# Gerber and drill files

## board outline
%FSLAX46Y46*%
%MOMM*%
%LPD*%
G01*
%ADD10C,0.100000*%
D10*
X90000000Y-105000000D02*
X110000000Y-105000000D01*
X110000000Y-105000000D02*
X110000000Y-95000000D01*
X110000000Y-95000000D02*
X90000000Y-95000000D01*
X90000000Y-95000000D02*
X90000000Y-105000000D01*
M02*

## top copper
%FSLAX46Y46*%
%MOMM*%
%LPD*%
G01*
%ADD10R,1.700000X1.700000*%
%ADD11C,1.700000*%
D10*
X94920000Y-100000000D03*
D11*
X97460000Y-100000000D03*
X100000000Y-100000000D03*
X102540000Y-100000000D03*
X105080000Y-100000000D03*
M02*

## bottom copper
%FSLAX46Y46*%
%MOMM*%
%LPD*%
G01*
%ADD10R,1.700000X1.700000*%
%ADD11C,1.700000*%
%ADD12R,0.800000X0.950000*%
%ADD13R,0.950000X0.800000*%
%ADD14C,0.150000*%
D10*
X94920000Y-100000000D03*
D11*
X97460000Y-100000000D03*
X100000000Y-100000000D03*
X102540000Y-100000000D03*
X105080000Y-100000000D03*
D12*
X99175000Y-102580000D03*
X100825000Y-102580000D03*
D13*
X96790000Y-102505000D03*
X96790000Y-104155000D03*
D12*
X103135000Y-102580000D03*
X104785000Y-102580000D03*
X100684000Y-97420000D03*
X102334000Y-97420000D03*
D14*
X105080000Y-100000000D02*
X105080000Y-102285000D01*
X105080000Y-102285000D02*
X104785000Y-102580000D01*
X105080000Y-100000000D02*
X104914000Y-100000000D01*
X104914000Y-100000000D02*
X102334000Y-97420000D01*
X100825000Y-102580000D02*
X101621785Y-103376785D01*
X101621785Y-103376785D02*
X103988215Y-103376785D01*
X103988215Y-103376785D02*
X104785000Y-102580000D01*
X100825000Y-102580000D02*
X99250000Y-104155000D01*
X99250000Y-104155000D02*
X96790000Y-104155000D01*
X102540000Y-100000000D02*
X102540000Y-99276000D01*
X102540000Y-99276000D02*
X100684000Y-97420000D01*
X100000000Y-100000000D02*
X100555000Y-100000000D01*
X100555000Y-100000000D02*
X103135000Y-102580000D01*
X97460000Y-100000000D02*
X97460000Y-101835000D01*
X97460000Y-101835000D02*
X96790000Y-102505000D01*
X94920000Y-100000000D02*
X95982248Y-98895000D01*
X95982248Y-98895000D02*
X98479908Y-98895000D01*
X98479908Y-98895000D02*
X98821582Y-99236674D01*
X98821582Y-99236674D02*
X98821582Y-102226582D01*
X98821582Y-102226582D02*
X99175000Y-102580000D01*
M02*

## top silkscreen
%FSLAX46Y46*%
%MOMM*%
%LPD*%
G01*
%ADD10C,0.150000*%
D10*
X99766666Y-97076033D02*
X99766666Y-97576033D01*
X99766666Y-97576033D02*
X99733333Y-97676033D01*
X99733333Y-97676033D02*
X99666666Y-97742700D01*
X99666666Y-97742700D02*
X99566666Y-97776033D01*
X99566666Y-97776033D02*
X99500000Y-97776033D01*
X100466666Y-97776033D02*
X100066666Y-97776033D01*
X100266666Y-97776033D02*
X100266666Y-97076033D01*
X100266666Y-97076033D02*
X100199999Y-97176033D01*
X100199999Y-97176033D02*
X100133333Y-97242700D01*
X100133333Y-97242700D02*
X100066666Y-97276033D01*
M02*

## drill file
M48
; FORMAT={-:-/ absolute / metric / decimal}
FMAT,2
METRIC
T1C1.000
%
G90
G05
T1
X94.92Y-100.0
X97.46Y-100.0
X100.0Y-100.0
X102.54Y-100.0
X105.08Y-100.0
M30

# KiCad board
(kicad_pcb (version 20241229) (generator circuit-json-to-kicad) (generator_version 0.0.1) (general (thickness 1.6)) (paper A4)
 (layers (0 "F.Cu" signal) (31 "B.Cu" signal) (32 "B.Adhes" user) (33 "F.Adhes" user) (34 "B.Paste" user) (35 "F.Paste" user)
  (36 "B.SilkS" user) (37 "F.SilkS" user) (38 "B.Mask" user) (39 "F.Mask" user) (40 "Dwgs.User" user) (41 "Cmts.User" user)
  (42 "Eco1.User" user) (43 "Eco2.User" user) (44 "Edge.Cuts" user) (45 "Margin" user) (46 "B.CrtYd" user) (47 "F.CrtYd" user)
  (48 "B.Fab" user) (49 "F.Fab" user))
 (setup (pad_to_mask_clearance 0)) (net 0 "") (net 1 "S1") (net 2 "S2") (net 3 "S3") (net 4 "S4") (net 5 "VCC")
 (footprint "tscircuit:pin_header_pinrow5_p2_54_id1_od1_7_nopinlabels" (layer F.Cu) (at 100 100 0)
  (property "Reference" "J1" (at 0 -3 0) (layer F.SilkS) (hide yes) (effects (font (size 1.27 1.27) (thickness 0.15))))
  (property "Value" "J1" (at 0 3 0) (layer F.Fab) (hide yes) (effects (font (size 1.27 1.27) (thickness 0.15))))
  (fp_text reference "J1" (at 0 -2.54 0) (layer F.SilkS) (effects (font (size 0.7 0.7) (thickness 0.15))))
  (pad "1" thru_hole rect (at -5.08 0 0) (size 1.7 1.7) (drill 1) (layers *.Cu *.Mask) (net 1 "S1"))
  (pad "2" thru_hole circle (at -2.54 0 0) (size 1.7 1.7) (drill 1) (layers *.Cu *.Mask) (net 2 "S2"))
  (pad "3" thru_hole circle (at 0 0 0) (size 1.7 1.7) (drill 1) (layers *.Cu *.Mask) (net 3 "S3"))
  (pad "4" thru_hole circle (at 2.54 0 0) (size 1.7 1.7) (drill 1) (layers *.Cu *.Mask) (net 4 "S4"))
  (pad "5" thru_hole circle (at 5.08 0 0) (size 1.7 1.7) (drill 1) (layers *.Cu *.Mask) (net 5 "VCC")))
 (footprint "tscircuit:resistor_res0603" (layer B.Cu) (at 100 102.58 180)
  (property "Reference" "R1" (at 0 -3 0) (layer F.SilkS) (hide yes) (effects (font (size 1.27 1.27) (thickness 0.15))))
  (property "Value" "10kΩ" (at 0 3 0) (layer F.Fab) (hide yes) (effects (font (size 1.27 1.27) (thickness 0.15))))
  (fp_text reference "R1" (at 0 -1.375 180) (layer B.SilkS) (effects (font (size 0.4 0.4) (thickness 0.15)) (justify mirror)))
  (pad "1" smd rect (at 0.825 0 0) (size 0.8 0.95) (layers B.Cu B.Mask) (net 1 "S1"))
  (pad "2" smd rect (at -0.825 0 0) (size 0.8 0.95) (layers B.Cu B.Mask) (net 5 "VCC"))
  (pad "" smd rect (at 0.825 0 0) (size 0.5599999999999999 0.6649999999999999) (layers B.Paste))
  (pad "" smd rect (at -0.825 0 0) (size 0.5599999999999999 0.6649999999999999) (layers B.Paste)))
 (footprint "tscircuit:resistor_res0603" (layer B.Cu) (at 96.79 103.33 90)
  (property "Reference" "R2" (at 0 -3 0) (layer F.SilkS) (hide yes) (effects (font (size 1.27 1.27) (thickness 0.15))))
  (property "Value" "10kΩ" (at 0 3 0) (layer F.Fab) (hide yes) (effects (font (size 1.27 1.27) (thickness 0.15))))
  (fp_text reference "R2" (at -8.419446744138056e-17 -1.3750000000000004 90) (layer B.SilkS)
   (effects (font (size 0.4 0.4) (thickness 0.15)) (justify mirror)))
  (pad "1" smd rect (at 0.8249999999999997 0 0) (size 0.95 0.8) (layers B.Cu B.Mask) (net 2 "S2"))
  (pad "2" smd rect (at -0.8249999999999997 4.440892098500626e-16 0) (size 0.95 0.8) (layers B.Cu B.Mask) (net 5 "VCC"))
  (pad "" smd rect (at 0.8249999999999997 0 0) (size 0.6649999999999999 0.5599999999999999) (layers B.Paste))
  (pad "" smd rect (at -0.8249999999999997 4.440892098500626e-16 0) (size 0.6649999999999999 0.5599999999999999) (layers B.Paste)))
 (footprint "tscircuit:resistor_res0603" (layer B.Cu) (at 103.96 102.58 180)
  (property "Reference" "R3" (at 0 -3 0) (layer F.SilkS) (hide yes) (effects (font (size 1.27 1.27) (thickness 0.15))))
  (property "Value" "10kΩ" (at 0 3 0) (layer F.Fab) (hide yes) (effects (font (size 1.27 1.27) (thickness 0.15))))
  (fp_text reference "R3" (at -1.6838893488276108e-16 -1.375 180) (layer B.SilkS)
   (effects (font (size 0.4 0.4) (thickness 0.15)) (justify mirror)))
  (pad "1" smd rect (at 0.8250000000000002 0 0) (size 0.8 0.95) (layers B.Cu B.Mask) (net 3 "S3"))
  (pad "2" smd rect (at -0.8249999999999997 0 0) (size 0.8 0.95) (layers B.Cu B.Mask) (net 5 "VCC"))
  (pad "" smd rect (at 0.8250000000000002 0 0) (size 0.5599999999999999 0.6649999999999999) (layers B.Paste))
  (pad "" smd rect (at -0.8249999999999997 0 0) (size 0.5599999999999999 0.6649999999999999) (layers B.Paste)))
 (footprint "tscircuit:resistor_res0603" (layer B.Cu) (at 101.509 97.42 180)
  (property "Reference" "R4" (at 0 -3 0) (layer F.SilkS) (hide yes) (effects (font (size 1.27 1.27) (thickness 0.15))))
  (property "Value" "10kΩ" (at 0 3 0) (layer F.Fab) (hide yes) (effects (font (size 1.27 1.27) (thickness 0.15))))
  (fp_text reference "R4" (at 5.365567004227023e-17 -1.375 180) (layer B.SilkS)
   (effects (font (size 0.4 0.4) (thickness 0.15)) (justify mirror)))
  (pad "1" smd rect (at 0.8250000000000001 0 0) (size 0.8 0.95) (layers B.Cu B.Mask) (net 4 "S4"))
  (pad "2" smd rect (at -0.825 4.440892098500626e-16 0) (size 0.8 0.95) (layers B.Cu B.Mask) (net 5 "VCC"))
  (pad "" smd rect (at 0.8250000000000001 0 0) (size 0.5599999999999999 0.6649999999999999) (layers B.Paste))
  (pad "" smd rect (at -0.825 4.440892098500626e-16 0) (size 0.5599999999999999 0.6649999999999999) (layers B.Paste)))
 (segment (start 105.08 100) (end 105.08 102.285) (width 0.15) (layer B.Cu) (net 5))
 (segment (start 105.08 102.285) (end 104.785 102.58) (width 0.15) (layer B.Cu) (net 5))
 (segment (start 105.08 100) (end 104.914 100) (width 0.15) (layer B.Cu) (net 5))
 (segment (start 104.914 100) (end 102.334 97.42) (width 0.15) (layer B.Cu) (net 5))
 (segment (start 100.825 102.58) (end 101.62178503083923 103.37678503083924) (width 0.15) (layer B.Cu) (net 5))
 (segment (start 101.62178503083923 103.37678503083924) (end 103.98821496916077 103.37678503083924) (width 0.15) (layer B.Cu) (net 5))
 (segment (start 103.98821496916077 103.37678503083924) (end 104.785 102.58) (width 0.15) (layer B.Cu) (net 5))
 (segment (start 100.825 102.58) (end 99.25 104.155) (width 0.15) (layer B.Cu) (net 5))
 (segment (start 99.25 104.155) (end 96.79 104.155) (width 0.15) (layer B.Cu) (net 5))
 (segment (start 102.54 100) (end 102.54 99.276) (width 0.15) (layer B.Cu) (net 4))
 (segment (start 102.54 99.276) (end 100.684 97.42) (width 0.15) (layer B.Cu) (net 4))
 (segment (start 100 100) (end 100.555 100) (width 0.15) (layer B.Cu) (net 3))
 (segment (start 100.555 100) (end 103.135 102.58) (width 0.15) (layer B.Cu) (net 3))
 (segment (start 97.46 100) (end 97.46 101.835) (width 0.15) (layer B.Cu) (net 2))
 (segment (start 97.46 101.835) (end 96.79 102.505) (width 0.15) (layer B.Cu) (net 2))
 (segment (start 94.92 100) (end 95.98224762684069 98.895) (width 0.15) (layer B.Cu) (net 1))
 (segment (start 95.98224762684069 98.895) (end 98.479907924164 98.895) (width 0.15) (layer B.Cu) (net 1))
 (segment (start 98.479907924164 98.895) (end 98.8215816032488 99.2366736790848) (width 0.15) (layer B.Cu) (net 1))
 (segment (start 98.8215816032488 99.2366736790848) (end 98.8215816032488 102.22658160324879) (width 0.15) (layer B.Cu) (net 1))
 (segment (start 98.8215816032488 102.22658160324879) (end 99.175 102.58) (width 0.15) (layer B.Cu) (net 1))
 (gr_line (start 90 105) (end 110 105) (width 0.1) (layer Edge.Cuts))
 (gr_line (start 110 105) (end 110 95) (width 0.1) (layer Edge.Cuts))
 (gr_line (start 110 95) (end 90 95) (width 0.1) (layer Edge.Cuts))
 (gr_line (start 90 95) (end 90 105) (width 0.1) (layer Edge.Cuts)))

